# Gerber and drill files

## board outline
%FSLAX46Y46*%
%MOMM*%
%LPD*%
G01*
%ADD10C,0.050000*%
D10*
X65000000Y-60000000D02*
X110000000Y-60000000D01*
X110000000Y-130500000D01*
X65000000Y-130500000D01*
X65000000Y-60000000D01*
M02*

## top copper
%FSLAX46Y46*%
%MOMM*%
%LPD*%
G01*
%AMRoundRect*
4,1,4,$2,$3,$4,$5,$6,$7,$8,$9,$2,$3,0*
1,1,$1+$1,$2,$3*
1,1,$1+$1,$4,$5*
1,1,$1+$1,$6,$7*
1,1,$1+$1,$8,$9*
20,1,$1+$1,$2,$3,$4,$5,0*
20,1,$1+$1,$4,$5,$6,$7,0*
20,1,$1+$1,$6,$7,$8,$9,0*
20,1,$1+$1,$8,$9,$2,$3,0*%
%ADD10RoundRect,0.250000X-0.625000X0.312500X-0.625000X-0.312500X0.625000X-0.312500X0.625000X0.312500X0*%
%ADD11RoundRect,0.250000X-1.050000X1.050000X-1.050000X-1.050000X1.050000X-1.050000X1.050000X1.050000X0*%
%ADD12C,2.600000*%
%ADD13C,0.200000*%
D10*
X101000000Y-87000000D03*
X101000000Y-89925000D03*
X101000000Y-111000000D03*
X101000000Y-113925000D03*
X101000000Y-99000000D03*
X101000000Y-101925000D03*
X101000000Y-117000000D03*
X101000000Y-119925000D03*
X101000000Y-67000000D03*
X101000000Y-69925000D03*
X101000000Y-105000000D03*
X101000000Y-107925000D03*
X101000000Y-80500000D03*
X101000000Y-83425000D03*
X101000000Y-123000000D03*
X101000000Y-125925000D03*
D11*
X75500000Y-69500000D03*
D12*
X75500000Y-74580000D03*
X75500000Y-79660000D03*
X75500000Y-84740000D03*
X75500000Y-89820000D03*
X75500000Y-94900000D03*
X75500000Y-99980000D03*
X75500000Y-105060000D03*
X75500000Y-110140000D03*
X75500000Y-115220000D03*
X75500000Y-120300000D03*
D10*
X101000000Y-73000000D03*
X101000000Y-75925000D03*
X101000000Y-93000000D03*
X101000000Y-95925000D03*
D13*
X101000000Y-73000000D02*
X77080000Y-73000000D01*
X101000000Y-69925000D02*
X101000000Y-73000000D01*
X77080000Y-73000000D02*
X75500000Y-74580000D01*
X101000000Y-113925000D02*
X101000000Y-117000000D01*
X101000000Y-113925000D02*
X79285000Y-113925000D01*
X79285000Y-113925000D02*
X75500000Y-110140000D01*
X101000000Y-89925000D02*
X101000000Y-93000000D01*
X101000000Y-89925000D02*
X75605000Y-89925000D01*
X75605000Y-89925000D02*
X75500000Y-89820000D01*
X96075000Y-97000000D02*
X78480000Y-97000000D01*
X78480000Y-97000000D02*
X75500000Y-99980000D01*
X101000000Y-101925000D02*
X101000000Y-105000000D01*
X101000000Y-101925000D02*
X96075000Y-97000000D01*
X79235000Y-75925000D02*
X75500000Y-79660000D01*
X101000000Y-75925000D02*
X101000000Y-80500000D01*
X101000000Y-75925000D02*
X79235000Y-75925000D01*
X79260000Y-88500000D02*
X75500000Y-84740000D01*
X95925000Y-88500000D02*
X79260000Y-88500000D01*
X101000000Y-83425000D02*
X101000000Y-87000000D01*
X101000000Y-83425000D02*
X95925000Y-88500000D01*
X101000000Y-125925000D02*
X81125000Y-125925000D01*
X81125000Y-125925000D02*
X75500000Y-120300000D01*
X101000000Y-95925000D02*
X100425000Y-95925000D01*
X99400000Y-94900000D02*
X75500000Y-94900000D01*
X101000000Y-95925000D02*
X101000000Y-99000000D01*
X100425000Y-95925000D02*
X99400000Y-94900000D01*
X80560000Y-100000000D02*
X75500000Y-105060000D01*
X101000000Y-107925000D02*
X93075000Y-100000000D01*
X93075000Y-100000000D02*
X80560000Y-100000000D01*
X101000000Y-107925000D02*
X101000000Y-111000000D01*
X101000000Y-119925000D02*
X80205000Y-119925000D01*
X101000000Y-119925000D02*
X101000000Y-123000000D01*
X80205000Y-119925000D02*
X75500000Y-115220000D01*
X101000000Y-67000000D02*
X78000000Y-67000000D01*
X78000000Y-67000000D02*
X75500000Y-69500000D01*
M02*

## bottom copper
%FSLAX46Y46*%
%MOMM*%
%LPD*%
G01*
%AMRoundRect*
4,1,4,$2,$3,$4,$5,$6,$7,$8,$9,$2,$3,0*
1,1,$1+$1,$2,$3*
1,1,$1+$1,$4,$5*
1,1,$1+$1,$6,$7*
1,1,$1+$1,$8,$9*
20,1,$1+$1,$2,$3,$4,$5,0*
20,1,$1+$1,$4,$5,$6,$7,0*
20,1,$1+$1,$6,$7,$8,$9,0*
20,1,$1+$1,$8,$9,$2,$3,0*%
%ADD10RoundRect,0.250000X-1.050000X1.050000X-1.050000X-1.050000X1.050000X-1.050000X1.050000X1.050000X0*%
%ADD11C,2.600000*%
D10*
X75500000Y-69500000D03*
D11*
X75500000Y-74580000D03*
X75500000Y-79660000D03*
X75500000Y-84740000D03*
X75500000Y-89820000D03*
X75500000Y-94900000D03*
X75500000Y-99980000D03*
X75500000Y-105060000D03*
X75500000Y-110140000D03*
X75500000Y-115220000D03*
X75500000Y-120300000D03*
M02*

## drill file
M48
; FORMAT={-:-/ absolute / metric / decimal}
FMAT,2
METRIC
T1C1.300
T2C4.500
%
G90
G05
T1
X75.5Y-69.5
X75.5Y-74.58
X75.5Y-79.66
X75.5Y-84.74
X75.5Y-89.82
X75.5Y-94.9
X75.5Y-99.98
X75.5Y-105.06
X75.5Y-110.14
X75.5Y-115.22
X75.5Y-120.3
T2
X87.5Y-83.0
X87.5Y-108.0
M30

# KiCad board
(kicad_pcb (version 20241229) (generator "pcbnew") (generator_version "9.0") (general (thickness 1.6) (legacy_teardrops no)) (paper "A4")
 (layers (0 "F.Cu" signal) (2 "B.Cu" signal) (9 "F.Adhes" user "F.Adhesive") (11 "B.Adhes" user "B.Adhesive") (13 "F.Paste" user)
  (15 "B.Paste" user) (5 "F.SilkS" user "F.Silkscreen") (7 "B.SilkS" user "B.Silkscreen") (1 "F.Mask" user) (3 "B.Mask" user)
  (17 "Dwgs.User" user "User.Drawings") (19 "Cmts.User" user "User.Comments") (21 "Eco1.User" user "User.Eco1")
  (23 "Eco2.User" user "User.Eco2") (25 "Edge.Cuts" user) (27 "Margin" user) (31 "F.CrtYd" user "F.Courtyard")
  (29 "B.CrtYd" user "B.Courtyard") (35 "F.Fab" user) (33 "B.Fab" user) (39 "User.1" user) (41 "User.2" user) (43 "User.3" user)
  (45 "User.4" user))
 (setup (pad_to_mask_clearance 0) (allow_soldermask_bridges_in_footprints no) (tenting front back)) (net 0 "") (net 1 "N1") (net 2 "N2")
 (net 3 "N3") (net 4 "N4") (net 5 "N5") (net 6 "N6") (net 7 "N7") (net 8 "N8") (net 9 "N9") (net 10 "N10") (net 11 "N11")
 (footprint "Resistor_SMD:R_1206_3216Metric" (layer "F.Cu") (at 101 88.4625 -90)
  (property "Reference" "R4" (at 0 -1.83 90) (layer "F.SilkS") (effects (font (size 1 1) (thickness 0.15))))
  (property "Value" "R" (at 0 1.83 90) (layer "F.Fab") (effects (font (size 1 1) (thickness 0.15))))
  (pad "1" smd roundrect (at -1.4625 0 270) (size 1.125 1.75) (layers "F.Cu" "F.Mask" "F.Paste") (roundrect_rratio 0.222222) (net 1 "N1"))
  (pad "2" smd roundrect (at 1.4625 0 270) (size 1.125 1.75) (layers "F.Cu" "F.Mask" "F.Paste") (roundrect_rratio 0.222222) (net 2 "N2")))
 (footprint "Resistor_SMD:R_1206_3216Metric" (layer "F.Cu") (at 101 112.4625 -90)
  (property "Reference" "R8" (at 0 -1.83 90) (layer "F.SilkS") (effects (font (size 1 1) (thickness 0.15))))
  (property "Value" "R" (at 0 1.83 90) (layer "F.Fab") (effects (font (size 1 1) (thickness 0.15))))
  (pad "1" smd roundrect (at -1.4625 0 270) (size 1.125 1.75) (layers "F.Cu" "F.Mask" "F.Paste") (roundrect_rratio 0.222222) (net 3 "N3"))
  (pad "2" smd roundrect (at 1.4625 0 270) (size 1.125 1.75) (layers "F.Cu" "F.Mask" "F.Paste") (roundrect_rratio 0.222222) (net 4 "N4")))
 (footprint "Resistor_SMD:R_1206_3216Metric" (layer "F.Cu") (at 101 100.4625 -90)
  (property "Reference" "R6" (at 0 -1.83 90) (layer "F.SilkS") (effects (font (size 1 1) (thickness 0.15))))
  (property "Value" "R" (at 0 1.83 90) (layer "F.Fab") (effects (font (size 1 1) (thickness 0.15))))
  (pad "1" smd roundrect (at -1.4625 0 270) (size 1.125 1.75) (layers "F.Cu" "F.Mask" "F.Paste") (roundrect_rratio 0.222222) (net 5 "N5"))
  (pad "2" smd roundrect (at 1.4625 0 270) (size 1.125 1.75) (layers "F.Cu" "F.Mask" "F.Paste") (roundrect_rratio 0.222222) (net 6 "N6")))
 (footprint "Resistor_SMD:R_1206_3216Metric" (layer "F.Cu") (at 101 118.4625 -90)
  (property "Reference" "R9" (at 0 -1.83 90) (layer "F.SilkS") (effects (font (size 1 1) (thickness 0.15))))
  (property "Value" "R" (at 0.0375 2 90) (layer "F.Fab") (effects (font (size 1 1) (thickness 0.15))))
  (pad "1" smd roundrect (at -1.4625 0 270) (size 1.125 1.75) (layers "F.Cu" "F.Mask" "F.Paste") (roundrect_rratio 0.222222) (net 4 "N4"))
  (pad "2" smd roundrect (at 1.4625 0 270) (size 1.125 1.75) (layers "F.Cu" "F.Mask" "F.Paste") (roundrect_rratio 0.222222) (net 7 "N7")))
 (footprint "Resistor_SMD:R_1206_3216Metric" (layer "F.Cu") (at 101 68.4625 -90)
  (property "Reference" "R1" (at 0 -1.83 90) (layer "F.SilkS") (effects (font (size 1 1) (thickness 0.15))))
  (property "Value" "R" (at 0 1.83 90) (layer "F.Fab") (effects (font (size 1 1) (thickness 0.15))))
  (pad "1" smd roundrect (at -1.4625 0 270) (size 1.125 1.75) (layers "F.Cu" "F.Mask" "F.Paste") (roundrect_rratio 0.222222) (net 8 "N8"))
  (pad "2" smd roundrect (at 1.4625 0 270) (size 1.125 1.75) (layers "F.Cu" "F.Mask" "F.Paste") (roundrect_rratio 0.222222) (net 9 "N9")))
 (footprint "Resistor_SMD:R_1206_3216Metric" (layer "F.Cu") (at 101 106.4625 -90)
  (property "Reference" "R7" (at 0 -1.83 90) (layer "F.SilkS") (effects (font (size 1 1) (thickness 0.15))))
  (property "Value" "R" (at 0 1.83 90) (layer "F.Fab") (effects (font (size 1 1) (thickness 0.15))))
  (pad "1" smd roundrect (at -1.4625 0 270) (size 1.125 1.75) (layers "F.Cu" "F.Mask" "F.Paste") (roundrect_rratio 0.222222) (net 6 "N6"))
  (pad "2" smd roundrect (at 1.4625 0 270) (size 1.125 1.75) (layers "F.Cu" "F.Mask" "F.Paste") (roundrect_rratio 0.222222) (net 3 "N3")))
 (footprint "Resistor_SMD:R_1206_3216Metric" (layer "F.Cu") (at 101 81.9625 -90)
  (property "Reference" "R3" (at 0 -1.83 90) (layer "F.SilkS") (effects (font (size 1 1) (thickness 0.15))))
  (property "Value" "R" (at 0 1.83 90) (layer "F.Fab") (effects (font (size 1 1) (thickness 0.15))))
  (pad "1" smd roundrect (at -1.4625 0 270) (size 1.125 1.75) (layers "F.Cu" "F.Mask" "F.Paste") (roundrect_rratio 0.222222) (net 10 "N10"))
  (pad "2" smd roundrect (at 1.4625 0 270) (size 1.125 1.75) (layers "F.Cu" "F.Mask" "F.Paste") (roundrect_rratio 0.222222) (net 1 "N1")))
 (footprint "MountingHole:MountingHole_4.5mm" (layer "F.Cu") (at 87.5 83)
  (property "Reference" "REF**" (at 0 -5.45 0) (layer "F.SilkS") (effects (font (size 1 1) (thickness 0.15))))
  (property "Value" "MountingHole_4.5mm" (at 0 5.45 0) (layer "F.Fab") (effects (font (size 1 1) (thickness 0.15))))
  (pad "" np_thru_hole circle (at 0 0) (size 4.5 4.5) (drill 4.5) (layers "*.Cu" "*.Mask")))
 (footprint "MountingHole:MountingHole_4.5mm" (layer "F.Cu") (at 87.5 108)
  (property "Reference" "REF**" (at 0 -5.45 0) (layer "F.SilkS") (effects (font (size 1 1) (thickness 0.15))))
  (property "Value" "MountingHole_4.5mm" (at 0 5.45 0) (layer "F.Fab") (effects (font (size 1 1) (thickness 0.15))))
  (pad "" np_thru_hole circle (at 0 0) (size 4.5 4.5) (drill 4.5) (layers "*.Cu" "*.Mask")))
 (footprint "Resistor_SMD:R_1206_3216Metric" (layer "F.Cu") (at 101 124.4625 -90)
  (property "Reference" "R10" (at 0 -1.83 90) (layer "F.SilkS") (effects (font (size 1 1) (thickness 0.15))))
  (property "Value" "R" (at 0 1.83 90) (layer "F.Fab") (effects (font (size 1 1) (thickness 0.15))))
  (pad "1" smd roundrect (at -1.4625 0 270) (size 1.125 1.75) (layers "F.Cu" "F.Mask" "F.Paste") (roundrect_rratio 0.222222) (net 7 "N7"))
  (pad "2" smd roundrect (at 1.4625 0 270) (size 1.125 1.75) (layers "F.Cu" "F.Mask" "F.Paste") (roundrect_rratio 0.222222) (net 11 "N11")))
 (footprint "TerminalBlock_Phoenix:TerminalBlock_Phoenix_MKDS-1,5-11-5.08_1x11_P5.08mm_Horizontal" (layer "F.Cu") (at 75.5 69.5 -90)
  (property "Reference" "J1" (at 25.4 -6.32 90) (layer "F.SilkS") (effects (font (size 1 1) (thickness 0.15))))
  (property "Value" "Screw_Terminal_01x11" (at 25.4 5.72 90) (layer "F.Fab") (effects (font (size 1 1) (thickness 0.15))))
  (pad "1" thru_hole roundrect (at 0 0 270) (size 2.6 2.6) (drill 1.3) (layers "*.Cu" "*.Mask") (remove_unused_layers no)
   (roundrect_rratio 0.096154) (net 8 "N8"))
  (pad "2" thru_hole circle (at 5.08 0 270) (size 2.6 2.6) (drill 1.3) (layers "*.Cu" "*.Mask") (remove_unused_layers no) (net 9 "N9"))
  (pad "3" thru_hole circle (at 10.16 0 270) (size 2.6 2.6) (drill 1.3) (layers "*.Cu" "*.Mask") (remove_unused_layers no) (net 10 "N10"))
  (pad "4" thru_hole circle (at 15.24 0 270) (size 2.6 2.6) (drill 1.3) (layers "*.Cu" "*.Mask") (remove_unused_layers no) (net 1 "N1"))
  (pad "5" thru_hole circle (at 20.32 0 270) (size 2.6 2.6) (drill 1.3) (layers "*.Cu" "*.Mask") (remove_unused_layers no) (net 2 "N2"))
  (pad "6" thru_hole circle (at 25.4 0 270) (size 2.6 2.6) (drill 1.3) (layers "*.Cu" "*.Mask") (remove_unused_layers no) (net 5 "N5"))
  (pad "7" thru_hole circle (at 30.48 0 270) (size 2.6 2.6) (drill 1.3) (layers "*.Cu" "*.Mask") (remove_unused_layers no) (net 6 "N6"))
  (pad "8" thru_hole circle (at 35.56 0 270) (size 2.6 2.6) (drill 1.3) (layers "*.Cu" "*.Mask") (remove_unused_layers no) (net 3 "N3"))
  (pad "9" thru_hole circle (at 40.64 0 270) (size 2.6 2.6) (drill 1.3) (layers "*.Cu" "*.Mask") (remove_unused_layers no) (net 4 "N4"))
  (pad "10" thru_hole circle (at 45.72 0 270) (size 2.6 2.6) (drill 1.3) (layers "*.Cu" "*.Mask") (remove_unused_layers no) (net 7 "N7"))
  (pad "11" thru_hole circle (at 50.8 0 270) (size 2.6 2.6) (drill 1.3) (layers "*.Cu" "*.Mask") (remove_unused_layers no) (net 11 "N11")))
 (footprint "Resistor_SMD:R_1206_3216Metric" (layer "F.Cu") (at 101 74.4625 -90)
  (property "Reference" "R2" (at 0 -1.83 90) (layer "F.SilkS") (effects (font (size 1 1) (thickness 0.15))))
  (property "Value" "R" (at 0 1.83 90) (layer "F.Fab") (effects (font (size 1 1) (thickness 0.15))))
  (pad "1" smd roundrect (at -1.4625 0 270) (size 1.125 1.75) (layers "F.Cu" "F.Mask" "F.Paste") (roundrect_rratio 0.222222) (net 9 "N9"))
  (pad "2" smd roundrect (at 1.4625 0 270) (size 1.125 1.75) (layers "F.Cu" "F.Mask" "F.Paste") (roundrect_rratio 0.222222) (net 10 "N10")))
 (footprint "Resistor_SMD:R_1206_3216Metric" (layer "F.Cu") (at 101 94.4625 -90)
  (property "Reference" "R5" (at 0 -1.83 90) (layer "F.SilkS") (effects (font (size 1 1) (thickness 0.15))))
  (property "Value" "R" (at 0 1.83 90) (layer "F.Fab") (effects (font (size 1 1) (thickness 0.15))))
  (pad "1" smd roundrect (at -1.4625 0 270) (size 1.125 1.75) (layers "F.Cu" "F.Mask" "F.Paste") (roundrect_rratio 0.222222) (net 2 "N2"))
  (pad "2" smd roundrect (at 1.4625 0 270) (size 1.125 1.75) (layers "F.Cu" "F.Mask" "F.Paste") (roundrect_rratio 0.222222) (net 5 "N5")))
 (gr_rect (start 65 60) (end 110 130.5) (stroke (width 0.05) (type default)) (fill no) (layer "Edge.Cuts"))
 (segment (start 101 73) (end 77.08 73) (width 0.2) (layer "F.Cu") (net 9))
 (segment (start 101 69.925) (end 101 73) (width 0.2) (layer "F.Cu") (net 9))
 (segment (start 77.08 73) (end 75.5 74.58) (width 0.2) (layer "F.Cu") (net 9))
 (segment (start 101 113.925) (end 101 117) (width 0.2) (layer "F.Cu") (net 4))
 (segment (start 101 113.925) (end 79.285 113.925) (width 0.2) (layer "F.Cu") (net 4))
 (segment (start 79.285 113.925) (end 75.5 110.14) (width 0.2) (layer "F.Cu") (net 4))
 (segment (start 101 89.925) (end 101 93) (width 0.2) (layer "F.Cu") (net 2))
 (segment (start 101 89.925) (end 75.605 89.925) (width 0.2) (layer "F.Cu") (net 2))
 (segment (start 75.605 89.925) (end 75.5 89.82) (width 0.2) (layer "F.Cu") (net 2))
 (segment (start 96.075 97) (end 78.48 97) (width 0.2) (layer "F.Cu") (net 6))
 (segment (start 78.48 97) (end 75.5 99.98) (width 0.2) (layer "F.Cu") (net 6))
 (segment (start 101 101.925) (end 101 105) (width 0.2) (layer "F.Cu") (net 6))
 (segment (start 101 101.925) (end 96.075 97) (width 0.2) (layer "F.Cu") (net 6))
 (segment (start 79.235 75.925) (end 75.5 79.66) (width 0.2) (layer "F.Cu") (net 10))
 (segment (start 101 75.925) (end 101 80.5) (width 0.2) (layer "F.Cu") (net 10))
 (segment (start 101 75.925) (end 79.235 75.925) (width 0.2) (layer "F.Cu") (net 10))
 (segment (start 79.26 88.5) (end 75.5 84.74) (width 0.2) (layer "F.Cu") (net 1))
 (segment (start 95.925 88.5) (end 79.26 88.5) (width 0.2) (layer "F.Cu") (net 1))
 (segment (start 101 83.425) (end 101 87) (width 0.2) (layer "F.Cu") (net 1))
 (segment (start 101 83.425) (end 95.925 88.5) (width 0.2) (layer "F.Cu") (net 1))
 (segment (start 101 125.925) (end 81.125 125.925) (width 0.2) (layer "F.Cu") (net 11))
 (segment (start 81.125 125.925) (end 75.5 120.3) (width 0.2) (layer "F.Cu") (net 11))
 (segment (start 101 95.925) (end 100.425 95.925) (width 0.2) (layer "F.Cu") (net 5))
 (segment (start 99.4 94.9) (end 75.5 94.9) (width 0.2) (layer "F.Cu") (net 5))
 (segment (start 101 95.925) (end 101 99) (width 0.2) (layer "F.Cu") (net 5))
 (segment (start 100.425 95.925) (end 99.4 94.9) (width 0.2) (layer "F.Cu") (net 5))
 (segment (start 80.56 100) (end 75.5 105.06) (width 0.2) (layer "F.Cu") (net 3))
 (segment (start 101 107.925) (end 93.075 100) (width 0.2) (layer "F.Cu") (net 3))
 (segment (start 93.075 100) (end 80.56 100) (width 0.2) (layer "F.Cu") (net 3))
 (segment (start 101 107.925) (end 101 111) (width 0.2) (layer "F.Cu") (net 3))
 (segment (start 101 119.925) (end 80.205 119.925) (width 0.2) (layer "F.Cu") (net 7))
 (segment (start 101 119.925) (end 101 123) (width 0.2) (layer "F.Cu") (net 7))
 (segment (start 80.205 119.925) (end 75.5 115.22) (width 0.2) (layer "F.Cu") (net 7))
 (segment (start 101 67) (end 78 67) (width 0.2) (layer "F.Cu") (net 8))
 (segment (start 78 67) (end 75.5 69.5) (width 0.2) (layer "F.Cu") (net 8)))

